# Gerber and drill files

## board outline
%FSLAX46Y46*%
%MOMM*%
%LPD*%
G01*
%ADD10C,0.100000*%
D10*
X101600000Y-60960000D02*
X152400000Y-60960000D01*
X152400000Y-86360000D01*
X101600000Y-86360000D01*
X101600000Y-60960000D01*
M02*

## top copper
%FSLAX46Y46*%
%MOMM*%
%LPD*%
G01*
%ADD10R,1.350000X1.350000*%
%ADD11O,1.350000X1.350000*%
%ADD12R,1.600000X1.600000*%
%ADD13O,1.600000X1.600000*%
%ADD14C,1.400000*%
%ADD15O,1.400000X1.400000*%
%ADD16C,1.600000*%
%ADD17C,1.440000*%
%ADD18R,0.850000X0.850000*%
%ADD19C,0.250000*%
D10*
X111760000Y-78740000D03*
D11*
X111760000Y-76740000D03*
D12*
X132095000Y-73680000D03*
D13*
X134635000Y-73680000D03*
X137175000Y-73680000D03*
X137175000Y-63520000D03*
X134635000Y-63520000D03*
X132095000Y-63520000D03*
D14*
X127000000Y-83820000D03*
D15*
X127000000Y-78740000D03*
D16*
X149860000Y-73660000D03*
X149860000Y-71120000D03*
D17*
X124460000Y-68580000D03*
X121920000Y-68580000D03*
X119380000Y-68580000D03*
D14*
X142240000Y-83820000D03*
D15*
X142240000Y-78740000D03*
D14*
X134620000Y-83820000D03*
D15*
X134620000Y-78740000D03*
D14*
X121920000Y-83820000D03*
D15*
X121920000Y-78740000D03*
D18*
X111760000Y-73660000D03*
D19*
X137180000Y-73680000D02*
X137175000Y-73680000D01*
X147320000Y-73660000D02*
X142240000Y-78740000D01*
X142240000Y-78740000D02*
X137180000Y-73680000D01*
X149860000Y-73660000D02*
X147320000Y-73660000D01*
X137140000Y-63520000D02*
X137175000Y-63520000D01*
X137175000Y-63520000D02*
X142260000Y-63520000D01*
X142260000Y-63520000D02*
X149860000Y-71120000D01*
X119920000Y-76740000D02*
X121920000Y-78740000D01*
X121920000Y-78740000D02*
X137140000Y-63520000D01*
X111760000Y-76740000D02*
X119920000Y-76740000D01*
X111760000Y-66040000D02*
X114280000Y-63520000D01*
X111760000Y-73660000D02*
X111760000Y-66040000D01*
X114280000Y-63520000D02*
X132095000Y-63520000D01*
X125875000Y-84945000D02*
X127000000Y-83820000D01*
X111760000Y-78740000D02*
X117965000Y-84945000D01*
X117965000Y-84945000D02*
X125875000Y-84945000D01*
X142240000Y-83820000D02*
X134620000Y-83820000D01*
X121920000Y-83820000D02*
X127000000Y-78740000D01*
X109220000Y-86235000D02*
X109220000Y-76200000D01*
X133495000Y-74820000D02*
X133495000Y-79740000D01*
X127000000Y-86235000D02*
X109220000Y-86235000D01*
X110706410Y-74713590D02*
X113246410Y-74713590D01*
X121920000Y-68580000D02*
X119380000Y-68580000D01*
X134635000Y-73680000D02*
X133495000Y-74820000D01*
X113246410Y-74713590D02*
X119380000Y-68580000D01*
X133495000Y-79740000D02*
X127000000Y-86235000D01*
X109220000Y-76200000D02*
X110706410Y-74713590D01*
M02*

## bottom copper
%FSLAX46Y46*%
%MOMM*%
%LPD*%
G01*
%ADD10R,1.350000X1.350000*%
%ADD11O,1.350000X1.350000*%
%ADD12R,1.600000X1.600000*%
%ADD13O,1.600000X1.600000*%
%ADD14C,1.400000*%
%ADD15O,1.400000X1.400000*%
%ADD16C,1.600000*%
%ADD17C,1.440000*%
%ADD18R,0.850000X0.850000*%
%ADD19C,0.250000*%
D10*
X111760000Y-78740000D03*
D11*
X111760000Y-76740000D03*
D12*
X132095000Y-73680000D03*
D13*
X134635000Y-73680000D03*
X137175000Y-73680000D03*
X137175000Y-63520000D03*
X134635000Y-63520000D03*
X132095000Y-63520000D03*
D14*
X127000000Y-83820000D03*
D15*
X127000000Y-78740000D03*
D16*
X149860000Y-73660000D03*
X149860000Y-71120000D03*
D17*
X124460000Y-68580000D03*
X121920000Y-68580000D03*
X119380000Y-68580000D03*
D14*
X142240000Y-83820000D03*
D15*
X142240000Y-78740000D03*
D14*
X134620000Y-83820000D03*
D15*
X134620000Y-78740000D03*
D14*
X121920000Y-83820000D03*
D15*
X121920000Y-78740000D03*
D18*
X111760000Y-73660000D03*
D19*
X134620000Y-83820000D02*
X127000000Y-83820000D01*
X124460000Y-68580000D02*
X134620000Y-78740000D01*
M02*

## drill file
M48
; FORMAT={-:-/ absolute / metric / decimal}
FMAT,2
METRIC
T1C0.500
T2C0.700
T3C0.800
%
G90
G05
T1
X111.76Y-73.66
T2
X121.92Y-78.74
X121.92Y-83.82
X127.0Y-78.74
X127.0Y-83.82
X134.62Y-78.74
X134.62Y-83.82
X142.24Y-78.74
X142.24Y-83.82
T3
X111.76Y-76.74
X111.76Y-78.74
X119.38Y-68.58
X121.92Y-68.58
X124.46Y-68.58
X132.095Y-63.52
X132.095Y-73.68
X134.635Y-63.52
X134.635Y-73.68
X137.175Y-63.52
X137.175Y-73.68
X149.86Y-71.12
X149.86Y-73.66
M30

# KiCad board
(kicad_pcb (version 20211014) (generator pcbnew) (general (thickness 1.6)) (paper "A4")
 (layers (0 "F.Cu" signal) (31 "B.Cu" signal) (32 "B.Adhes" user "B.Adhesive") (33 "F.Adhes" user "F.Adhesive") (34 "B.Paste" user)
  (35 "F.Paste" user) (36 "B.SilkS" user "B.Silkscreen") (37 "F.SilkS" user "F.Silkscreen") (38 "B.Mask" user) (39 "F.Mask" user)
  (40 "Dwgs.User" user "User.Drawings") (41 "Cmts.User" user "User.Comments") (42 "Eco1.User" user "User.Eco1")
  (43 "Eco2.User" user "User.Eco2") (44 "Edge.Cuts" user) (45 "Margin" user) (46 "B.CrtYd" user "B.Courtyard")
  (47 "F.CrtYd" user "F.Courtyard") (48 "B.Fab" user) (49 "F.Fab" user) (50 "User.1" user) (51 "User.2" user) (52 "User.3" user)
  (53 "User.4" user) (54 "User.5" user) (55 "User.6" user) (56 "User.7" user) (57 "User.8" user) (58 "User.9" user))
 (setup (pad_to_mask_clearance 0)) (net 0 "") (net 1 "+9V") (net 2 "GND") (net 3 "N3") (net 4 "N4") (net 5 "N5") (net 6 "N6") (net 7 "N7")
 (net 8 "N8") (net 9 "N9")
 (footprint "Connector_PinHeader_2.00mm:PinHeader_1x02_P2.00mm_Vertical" (layer "F.Cu") (at 111.76 78.74 180)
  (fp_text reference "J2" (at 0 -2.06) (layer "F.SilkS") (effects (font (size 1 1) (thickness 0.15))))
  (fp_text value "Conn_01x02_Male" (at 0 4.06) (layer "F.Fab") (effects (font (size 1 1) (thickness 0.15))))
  (pad "1" thru_hole rect (at 0 0 180) (size 1.35 1.35) (drill 0.8) (layers *.Cu *.Mask) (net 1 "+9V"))
  (pad "2" thru_hole oval (at 0 2 180) (size 1.35 1.35) (drill 0.8) (layers *.Cu *.Mask) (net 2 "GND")))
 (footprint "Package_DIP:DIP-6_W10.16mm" (layer "F.Cu") (at 132.095 73.68 90)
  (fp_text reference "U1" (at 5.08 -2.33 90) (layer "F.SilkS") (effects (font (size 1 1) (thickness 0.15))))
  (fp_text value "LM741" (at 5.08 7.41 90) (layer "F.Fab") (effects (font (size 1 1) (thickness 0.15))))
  (pad "1" thru_hole rect (at 0 0 90) (size 1.6 1.6) (drill 0.8) (layers *.Cu *.Mask) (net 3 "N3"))
  (pad "2" thru_hole oval (at 0 2.54 90) (size 1.6 1.6) (drill 0.8) (layers *.Cu *.Mask) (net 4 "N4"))
  (pad "3" thru_hole oval (at 0 5.08 90) (size 1.6 1.6) (drill 0.8) (layers *.Cu *.Mask) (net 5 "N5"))
  (pad "4" thru_hole oval (at 10.16 5.08 90) (size 1.6 1.6) (drill 0.8) (layers *.Cu *.Mask) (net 2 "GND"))
  (pad "5" thru_hole oval (at 10.16 2.54 90) (size 1.6 1.6) (drill 0.8) (layers *.Cu *.Mask) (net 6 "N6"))
  (pad "6" thru_hole oval (at 10.16 0 90) (size 1.6 1.6) (drill 0.8) (layers *.Cu *.Mask) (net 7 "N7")))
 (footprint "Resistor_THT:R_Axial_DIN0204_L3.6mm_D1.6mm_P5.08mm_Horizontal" (layer "F.Cu") (at 127 83.82 90)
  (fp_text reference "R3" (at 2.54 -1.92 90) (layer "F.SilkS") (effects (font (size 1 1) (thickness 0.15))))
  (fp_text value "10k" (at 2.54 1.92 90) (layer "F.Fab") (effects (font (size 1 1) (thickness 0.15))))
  (pad "1" thru_hole circle (at 0 0 90) (size 1.4 1.4) (drill 0.7) (layers *.Cu *.Mask) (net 1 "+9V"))
  (pad "2" thru_hole oval (at 5.08 0 90) (size 1.4 1.4) (drill 0.7) (layers *.Cu *.Mask) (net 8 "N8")))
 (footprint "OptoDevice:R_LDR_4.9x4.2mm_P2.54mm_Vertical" (layer "F.Cu") (at 149.86 73.66 90)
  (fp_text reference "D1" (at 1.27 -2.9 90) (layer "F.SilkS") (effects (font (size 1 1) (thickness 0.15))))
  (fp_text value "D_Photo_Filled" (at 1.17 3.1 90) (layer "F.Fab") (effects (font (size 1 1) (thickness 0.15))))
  (pad "1" thru_hole circle (at 0 0 90) (size 1.6 1.6) (drill 0.8) (layers *.Cu *.Mask) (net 5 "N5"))
  (pad "2" thru_hole circle (at 2.54 0 90) (size 1.6 1.6) (drill 0.8) (layers *.Cu *.Mask) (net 2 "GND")))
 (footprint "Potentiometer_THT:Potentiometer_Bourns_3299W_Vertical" (layer "F.Cu") (at 124.46 68.58)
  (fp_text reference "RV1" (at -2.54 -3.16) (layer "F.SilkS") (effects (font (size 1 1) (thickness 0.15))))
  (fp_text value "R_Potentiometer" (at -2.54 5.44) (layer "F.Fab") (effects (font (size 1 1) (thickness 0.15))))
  (pad "1" thru_hole circle (at 0 0) (size 1.44 1.44) (drill 0.8) (layers *.Cu *.Mask) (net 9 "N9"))
  (pad "2" thru_hole circle (at -2.54 0) (size 1.44 1.44) (drill 0.8) (layers *.Cu *.Mask) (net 4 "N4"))
  (pad "3" thru_hole circle (at -5.08 0) (size 1.44 1.44) (drill 0.8) (layers *.Cu *.Mask) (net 4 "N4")))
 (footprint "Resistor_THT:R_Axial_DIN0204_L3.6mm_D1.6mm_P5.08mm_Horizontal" (layer "F.Cu") (at 142.24 83.82 90)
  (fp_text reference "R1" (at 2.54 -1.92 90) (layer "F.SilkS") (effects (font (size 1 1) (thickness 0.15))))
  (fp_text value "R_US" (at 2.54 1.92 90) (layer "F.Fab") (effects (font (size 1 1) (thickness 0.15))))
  (pad "1" thru_hole circle (at 0 0 90) (size 1.4 1.4) (drill 0.7) (layers *.Cu *.Mask) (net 1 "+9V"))
  (pad "2" thru_hole oval (at 5.08 0 90) (size 1.4 1.4) (drill 0.7) (layers *.Cu *.Mask) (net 5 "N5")))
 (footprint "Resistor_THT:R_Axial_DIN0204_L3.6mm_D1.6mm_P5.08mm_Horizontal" (layer "F.Cu") (at 134.62 83.82 90)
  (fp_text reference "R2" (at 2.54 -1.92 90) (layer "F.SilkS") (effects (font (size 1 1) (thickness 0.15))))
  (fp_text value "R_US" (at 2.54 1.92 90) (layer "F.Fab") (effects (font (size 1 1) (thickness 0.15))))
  (pad "1" thru_hole circle (at 0 0 90) (size 1.4 1.4) (drill 0.7) (layers *.Cu *.Mask) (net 1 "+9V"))
  (pad "2" thru_hole oval (at 5.08 0 90) (size 1.4 1.4) (drill 0.7) (layers *.Cu *.Mask) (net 9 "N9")))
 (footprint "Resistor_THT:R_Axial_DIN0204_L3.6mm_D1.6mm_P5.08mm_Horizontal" (layer "F.Cu") (at 121.92 83.82 90)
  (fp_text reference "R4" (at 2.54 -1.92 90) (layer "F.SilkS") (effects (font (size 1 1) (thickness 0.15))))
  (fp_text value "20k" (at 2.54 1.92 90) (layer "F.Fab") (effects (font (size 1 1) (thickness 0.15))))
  (pad "1" thru_hole circle (at 0 0 90) (size 1.4 1.4) (drill 0.7) (layers *.Cu *.Mask) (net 8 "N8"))
  (pad "2" thru_hole oval (at 5.08 0 90) (size 1.4 1.4) (drill 0.7) (layers *.Cu *.Mask) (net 2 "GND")))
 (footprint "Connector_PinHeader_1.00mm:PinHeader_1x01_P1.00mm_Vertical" (layer "F.Cu") (at 111.76 73.66)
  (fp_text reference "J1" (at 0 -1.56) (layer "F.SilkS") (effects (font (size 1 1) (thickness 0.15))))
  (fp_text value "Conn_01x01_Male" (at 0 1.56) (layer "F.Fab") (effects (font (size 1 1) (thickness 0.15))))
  (pad "1" thru_hole rect (at 0 0) (size 0.85 0.85) (drill 0.5) (layers *.Cu *.Mask) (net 7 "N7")))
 (gr_rect (start 101.6 60.96) (end 152.4 86.36) (layer "Edge.Cuts") (width 0.1) (fill none))
 (segment (start 137.18 73.68) (end 137.175 73.68) (width 0.25) (layer "F.Cu") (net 5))
 (segment (start 147.32 73.66) (end 142.24 78.74) (width 0.25) (layer "F.Cu") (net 5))
 (segment (start 142.24 78.74) (end 137.18 73.68) (width 0.25) (layer "F.Cu") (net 5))
 (segment (start 149.86 73.66) (end 147.32 73.66) (width 0.25) (layer "F.Cu") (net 5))
 (segment (start 137.14 63.52) (end 137.175 63.52) (width 0.25) (layer "F.Cu") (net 2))
 (segment (start 137.175 63.52) (end 142.26 63.52) (width 0.25) (layer "F.Cu") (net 2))
 (segment (start 142.26 63.52) (end 149.86 71.12) (width 0.25) (layer "F.Cu") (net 2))
 (segment (start 119.92 76.74) (end 121.92 78.74) (width 0.25) (layer "F.Cu") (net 2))
 (segment (start 121.92 78.74) (end 137.14 63.52) (width 0.25) (layer "F.Cu") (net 2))
 (segment (start 111.76 76.74) (end 119.92 76.74) (width 0.25) (layer "F.Cu") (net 2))
 (segment (start 111.76 66.04) (end 114.28 63.52) (width 0.25) (layer "F.Cu") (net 7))
 (segment (start 111.76 73.66) (end 111.76 66.04) (width 0.25) (layer "F.Cu") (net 7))
 (segment (start 114.28 63.52) (end 132.095 63.52) (width 0.25) (layer "F.Cu") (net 7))
 (segment (start 125.875 84.945) (end 127 83.82) (width 0.25) (layer "F.Cu") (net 1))
 (segment (start 111.76 78.74) (end 117.965 84.945) (width 0.25) (layer "F.Cu") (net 1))
 (segment (start 117.965 84.945) (end 125.875 84.945) (width 0.25) (layer "F.Cu") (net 1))
 (segment (start 142.24 83.82) (end 134.62 83.82) (width 0.25) (layer "F.Cu") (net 1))
 (segment (start 134.62 83.82) (end 127 83.82) (width 0.25) (layer "B.Cu") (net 1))
 (segment (start 124.46 68.58) (end 134.62 78.74) (width 0.25) (layer "B.Cu") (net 9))
 (segment (start 121.92 83.82) (end 127 78.74) (width 0.25) (layer "F.Cu") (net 8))
 (segment (start 109.22 86.235) (end 109.22 76.2) (width 0.25) (layer "F.Cu") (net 4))
 (segment (start 133.495 74.82) (end 133.495 79.74) (width 0.25) (layer "F.Cu") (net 4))
 (segment (start 127 86.235) (end 109.22 86.235) (width 0.25) (layer "F.Cu") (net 4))
 (segment (start 110.70641 74.71359) (end 113.24641 74.71359) (width 0.25) (layer "F.Cu") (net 4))
 (segment (start 121.92 68.58) (end 119.38 68.58) (width 0.25) (layer "F.Cu") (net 4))
 (segment (start 134.635 73.68) (end 133.495 74.82) (width 0.25) (layer "F.Cu") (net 4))
 (segment (start 113.24641 74.71359) (end 119.38 68.58) (width 0.25) (layer "F.Cu") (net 4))
 (segment (start 133.495 79.74) (end 127 86.235) (width 0.25) (layer "F.Cu") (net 4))
 (segment (start 109.22 76.2) (end 110.70641 74.71359) (width 0.25) (layer "F.Cu") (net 4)))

